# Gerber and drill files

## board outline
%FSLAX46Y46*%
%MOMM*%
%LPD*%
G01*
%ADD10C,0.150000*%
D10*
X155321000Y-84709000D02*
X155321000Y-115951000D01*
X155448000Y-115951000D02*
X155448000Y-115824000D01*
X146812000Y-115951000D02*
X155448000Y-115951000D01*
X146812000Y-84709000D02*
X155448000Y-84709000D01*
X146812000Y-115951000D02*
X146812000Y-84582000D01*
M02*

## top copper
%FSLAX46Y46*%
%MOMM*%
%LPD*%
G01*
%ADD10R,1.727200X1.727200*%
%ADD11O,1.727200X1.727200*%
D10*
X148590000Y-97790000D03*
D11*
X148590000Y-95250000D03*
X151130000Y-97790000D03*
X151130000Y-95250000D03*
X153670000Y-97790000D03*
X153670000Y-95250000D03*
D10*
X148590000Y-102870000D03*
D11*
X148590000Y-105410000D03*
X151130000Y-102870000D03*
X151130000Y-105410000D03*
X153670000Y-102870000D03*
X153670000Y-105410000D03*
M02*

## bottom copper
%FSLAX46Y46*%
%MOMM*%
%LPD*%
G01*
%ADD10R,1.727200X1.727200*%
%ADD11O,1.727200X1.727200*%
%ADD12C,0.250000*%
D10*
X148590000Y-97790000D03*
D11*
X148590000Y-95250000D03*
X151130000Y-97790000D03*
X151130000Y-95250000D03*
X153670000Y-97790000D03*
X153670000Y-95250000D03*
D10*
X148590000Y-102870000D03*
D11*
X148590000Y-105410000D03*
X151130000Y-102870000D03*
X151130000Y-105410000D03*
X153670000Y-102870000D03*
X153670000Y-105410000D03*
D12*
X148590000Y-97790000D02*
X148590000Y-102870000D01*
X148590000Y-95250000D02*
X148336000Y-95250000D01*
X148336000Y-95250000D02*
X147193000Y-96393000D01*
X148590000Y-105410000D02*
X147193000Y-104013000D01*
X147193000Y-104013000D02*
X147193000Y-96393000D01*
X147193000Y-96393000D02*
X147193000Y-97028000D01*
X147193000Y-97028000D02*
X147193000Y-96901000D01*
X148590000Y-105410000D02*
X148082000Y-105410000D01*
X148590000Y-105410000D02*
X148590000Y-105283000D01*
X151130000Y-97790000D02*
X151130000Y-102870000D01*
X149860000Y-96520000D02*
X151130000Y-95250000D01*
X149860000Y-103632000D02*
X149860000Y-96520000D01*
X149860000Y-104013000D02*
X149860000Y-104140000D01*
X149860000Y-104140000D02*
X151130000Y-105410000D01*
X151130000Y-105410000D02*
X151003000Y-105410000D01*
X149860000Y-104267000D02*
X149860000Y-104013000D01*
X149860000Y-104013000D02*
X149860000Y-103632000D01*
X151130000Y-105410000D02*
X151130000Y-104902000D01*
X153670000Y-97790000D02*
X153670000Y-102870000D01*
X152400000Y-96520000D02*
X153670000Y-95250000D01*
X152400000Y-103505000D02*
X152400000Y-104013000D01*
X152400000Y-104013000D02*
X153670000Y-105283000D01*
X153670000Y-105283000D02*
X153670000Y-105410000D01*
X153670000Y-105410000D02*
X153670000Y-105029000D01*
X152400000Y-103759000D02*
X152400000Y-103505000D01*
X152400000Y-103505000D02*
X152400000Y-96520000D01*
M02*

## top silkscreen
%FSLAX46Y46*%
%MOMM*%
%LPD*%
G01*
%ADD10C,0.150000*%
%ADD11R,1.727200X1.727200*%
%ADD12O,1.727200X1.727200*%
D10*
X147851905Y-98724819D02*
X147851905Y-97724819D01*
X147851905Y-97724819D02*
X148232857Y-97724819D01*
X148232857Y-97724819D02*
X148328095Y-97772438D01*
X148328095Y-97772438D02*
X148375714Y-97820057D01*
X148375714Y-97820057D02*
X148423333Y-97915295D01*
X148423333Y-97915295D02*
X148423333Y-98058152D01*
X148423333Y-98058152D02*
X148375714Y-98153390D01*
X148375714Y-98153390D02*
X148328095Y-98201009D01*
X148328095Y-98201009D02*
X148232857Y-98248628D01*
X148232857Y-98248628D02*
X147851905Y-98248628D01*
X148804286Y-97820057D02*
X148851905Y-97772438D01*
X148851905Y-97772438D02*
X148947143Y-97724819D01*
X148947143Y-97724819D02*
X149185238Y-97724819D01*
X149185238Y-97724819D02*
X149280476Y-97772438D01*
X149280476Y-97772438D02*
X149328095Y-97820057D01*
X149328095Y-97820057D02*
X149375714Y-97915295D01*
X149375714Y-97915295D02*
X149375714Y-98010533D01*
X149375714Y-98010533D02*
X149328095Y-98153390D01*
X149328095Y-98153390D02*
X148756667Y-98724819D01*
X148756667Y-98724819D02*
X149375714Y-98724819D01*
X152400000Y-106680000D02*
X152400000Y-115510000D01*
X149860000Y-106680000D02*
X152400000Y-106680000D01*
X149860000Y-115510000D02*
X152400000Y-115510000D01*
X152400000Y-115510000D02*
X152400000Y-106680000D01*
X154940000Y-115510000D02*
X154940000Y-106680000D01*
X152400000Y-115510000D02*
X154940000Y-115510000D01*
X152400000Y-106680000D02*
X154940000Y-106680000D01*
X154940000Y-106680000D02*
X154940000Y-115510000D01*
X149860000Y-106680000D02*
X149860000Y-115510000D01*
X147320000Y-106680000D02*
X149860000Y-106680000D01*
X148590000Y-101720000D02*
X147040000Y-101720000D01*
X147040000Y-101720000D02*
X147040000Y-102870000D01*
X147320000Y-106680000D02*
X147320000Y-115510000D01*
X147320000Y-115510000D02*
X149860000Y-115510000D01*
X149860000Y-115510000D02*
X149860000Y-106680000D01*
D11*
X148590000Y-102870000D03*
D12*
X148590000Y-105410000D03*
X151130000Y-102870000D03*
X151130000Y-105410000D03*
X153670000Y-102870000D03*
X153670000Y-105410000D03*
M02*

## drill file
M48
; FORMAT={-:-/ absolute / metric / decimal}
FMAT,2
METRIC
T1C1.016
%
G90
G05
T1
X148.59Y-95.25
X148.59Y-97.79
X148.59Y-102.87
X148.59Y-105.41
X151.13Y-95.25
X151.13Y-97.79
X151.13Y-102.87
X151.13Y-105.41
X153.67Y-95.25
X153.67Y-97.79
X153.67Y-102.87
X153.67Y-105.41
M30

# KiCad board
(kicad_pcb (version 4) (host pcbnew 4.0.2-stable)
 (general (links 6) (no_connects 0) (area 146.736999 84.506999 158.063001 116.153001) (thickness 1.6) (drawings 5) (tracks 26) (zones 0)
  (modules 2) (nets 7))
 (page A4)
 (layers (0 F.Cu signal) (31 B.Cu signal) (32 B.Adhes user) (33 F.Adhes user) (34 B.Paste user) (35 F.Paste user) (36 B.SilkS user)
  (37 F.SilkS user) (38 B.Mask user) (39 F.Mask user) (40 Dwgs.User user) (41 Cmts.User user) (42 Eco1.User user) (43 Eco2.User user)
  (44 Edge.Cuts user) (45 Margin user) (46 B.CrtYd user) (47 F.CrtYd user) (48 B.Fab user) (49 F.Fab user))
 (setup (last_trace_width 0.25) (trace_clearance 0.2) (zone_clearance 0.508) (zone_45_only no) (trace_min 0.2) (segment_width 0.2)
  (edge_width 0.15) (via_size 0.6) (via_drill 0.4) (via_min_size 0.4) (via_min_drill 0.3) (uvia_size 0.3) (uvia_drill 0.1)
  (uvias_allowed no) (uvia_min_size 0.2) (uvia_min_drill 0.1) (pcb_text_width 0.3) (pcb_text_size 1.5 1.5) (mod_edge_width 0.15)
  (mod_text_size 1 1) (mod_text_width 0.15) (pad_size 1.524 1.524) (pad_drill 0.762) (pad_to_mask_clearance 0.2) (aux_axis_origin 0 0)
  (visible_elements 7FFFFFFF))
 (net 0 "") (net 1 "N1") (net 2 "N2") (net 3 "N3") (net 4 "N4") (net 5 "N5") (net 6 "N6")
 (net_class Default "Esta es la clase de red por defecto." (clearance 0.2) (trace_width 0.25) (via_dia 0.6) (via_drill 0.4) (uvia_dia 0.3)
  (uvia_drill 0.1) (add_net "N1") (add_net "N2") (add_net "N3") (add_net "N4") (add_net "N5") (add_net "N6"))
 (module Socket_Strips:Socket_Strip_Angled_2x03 (layer B.Cu) (at 148.59 97.79)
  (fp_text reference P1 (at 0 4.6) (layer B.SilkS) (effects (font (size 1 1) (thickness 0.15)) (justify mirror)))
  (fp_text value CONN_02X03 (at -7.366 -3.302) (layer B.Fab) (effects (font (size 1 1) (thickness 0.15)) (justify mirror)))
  (pad 1 thru_hole rect (at 0 0) (size 1.7272 1.7272) (drill 1.016) (layers *.Cu *.Mask B.SilkS) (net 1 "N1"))
  (pad 2 thru_hole oval (at 0 -2.54) (size 1.7272 1.7272) (drill 1.016) (layers *.Cu *.Mask B.SilkS) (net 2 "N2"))
  (pad 3 thru_hole oval (at 2.54 0) (size 1.7272 1.7272) (drill 1.016) (layers *.Cu *.Mask B.SilkS) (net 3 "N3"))
  (pad 4 thru_hole oval (at 2.54 -2.54) (size 1.7272 1.7272) (drill 1.016) (layers *.Cu *.Mask B.SilkS) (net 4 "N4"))
  (pad 5 thru_hole oval (at 5.08 0) (size 1.7272 1.7272) (drill 1.016) (layers *.Cu *.Mask B.SilkS) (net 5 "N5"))
  (pad 6 thru_hole oval (at 5.08 -2.54) (size 1.7272 1.7272) (drill 1.016) (layers *.Cu *.Mask B.SilkS) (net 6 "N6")))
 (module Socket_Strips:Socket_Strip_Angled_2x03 (layer F.Cu) (at 148.59 102.87)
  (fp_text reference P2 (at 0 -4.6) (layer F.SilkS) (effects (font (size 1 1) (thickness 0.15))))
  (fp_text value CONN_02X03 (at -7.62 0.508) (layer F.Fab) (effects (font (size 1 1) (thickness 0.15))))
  (fp_line (start 3.81 3.81) (end 3.81 12.64) (layer F.SilkS) (width 0.15))
  (fp_line (start 1.27 3.81) (end 3.81 3.81) (layer F.SilkS) (width 0.15))
  (fp_line (start 1.27 12.64) (end 3.81 12.64) (layer F.SilkS) (width 0.15))
  (fp_line (start 3.81 12.64) (end 3.81 3.81) (layer F.SilkS) (width 0.15))
  (fp_line (start 6.35 12.64) (end 6.35 3.81) (layer F.SilkS) (width 0.15))
  (fp_line (start 3.81 12.64) (end 6.35 12.64) (layer F.SilkS) (width 0.15))
  (fp_line (start 3.81 3.81) (end 6.35 3.81) (layer F.SilkS) (width 0.15))
  (fp_line (start 6.35 3.81) (end 6.35 12.64) (layer F.SilkS) (width 0.15))
  (fp_line (start 1.27 3.81) (end 1.27 12.64) (layer F.SilkS) (width 0.15))
  (fp_line (start -1.27 3.81) (end 1.27 3.81) (layer F.SilkS) (width 0.15))
  (fp_line (start 0 -1.15) (end -1.55 -1.15) (layer F.SilkS) (width 0.15))
  (fp_line (start -1.55 -1.15) (end -1.55 0) (layer F.SilkS) (width 0.15))
  (fp_line (start -1.27 3.81) (end -1.27 12.64) (layer F.SilkS) (width 0.15))
  (fp_line (start -1.27 12.64) (end 1.27 12.64) (layer F.SilkS) (width 0.15))
  (fp_line (start 1.27 12.64) (end 1.27 3.81) (layer F.SilkS) (width 0.15))
  (pad 1 thru_hole rect (at 0 0) (size 1.7272 1.7272) (drill 1.016) (layers *.Cu *.Mask F.SilkS) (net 1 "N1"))
  (pad 2 thru_hole oval (at 0 2.54) (size 1.7272 1.7272) (drill 1.016) (layers *.Cu *.Mask F.SilkS) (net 2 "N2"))
  (pad 3 thru_hole oval (at 2.54 0) (size 1.7272 1.7272) (drill 1.016) (layers *.Cu *.Mask F.SilkS) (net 3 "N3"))
  (pad 4 thru_hole oval (at 2.54 2.54) (size 1.7272 1.7272) (drill 1.016) (layers *.Cu *.Mask F.SilkS) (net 4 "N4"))
  (pad 5 thru_hole oval (at 5.08 0) (size 1.7272 1.7272) (drill 1.016) (layers *.Cu *.Mask F.SilkS) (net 5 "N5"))
  (pad 6 thru_hole oval (at 5.08 2.54) (size 1.7272 1.7272) (drill 1.016) (layers *.Cu *.Mask F.SilkS) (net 6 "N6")))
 (gr_line (start 155.321 84.709) (end 155.321 115.951) (angle 90) (layer Edge.Cuts) (width 0.15))
 (gr_line (start 155.448 115.951) (end 155.448 115.824) (angle 90) (layer Edge.Cuts) (width 0.15))
 (gr_line (start 146.812 115.951) (end 155.448 115.951) (angle 90) (layer Edge.Cuts) (width 0.15))
 (gr_line (start 146.812 84.709) (end 155.448 84.709) (angle 90) (layer Edge.Cuts) (width 0.15))
 (gr_line (start 146.812 115.951) (end 146.812 84.582) (angle 90) (layer Edge.Cuts) (width 0.15))
 (segment (start 148.59 97.79) (end 148.59 102.87) (width 0.25) (layer B.Cu) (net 1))
 (segment (start 148.59 95.25) (end 148.336 95.25) (width 0.25) (layer B.Cu) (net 2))
 (segment (start 148.336 95.25) (end 147.193 96.393) (width 0.25) (layer B.Cu) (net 2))
 (segment (start 148.59 105.41) (end 147.193 104.013) (width 0.25) (layer B.Cu) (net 2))
 (segment (start 147.193 104.013) (end 147.193 96.393) (width 0.25) (layer B.Cu) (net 2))
 (segment (start 147.193 96.393) (end 147.193 97.028) (width 0.25) (layer B.Cu) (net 2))
 (segment (start 147.193 97.028) (end 147.193 96.901) (width 0.25) (layer B.Cu) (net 2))
 (segment (start 148.59 105.41) (end 148.082 105.41) (width 0.25) (layer B.Cu) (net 2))
 (segment (start 148.59 105.41) (end 148.59 105.283) (width 0.25) (layer B.Cu) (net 2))
 (segment (start 151.13 97.79) (end 151.13 102.87) (width 0.25) (layer B.Cu) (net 3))
 (segment (start 149.86 96.52) (end 151.13 95.25) (width 0.25) (layer B.Cu) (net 4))
 (segment (start 149.86 103.632) (end 149.86 96.52) (width 0.25) (layer B.Cu) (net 4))
 (segment (start 149.86 104.013) (end 149.86 104.14) (width 0.25) (layer B.Cu) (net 4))
 (segment (start 149.86 104.14) (end 151.13 105.41) (width 0.25) (layer B.Cu) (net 4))
 (segment (start 151.13 105.41) (end 151.003 105.41) (width 0.25) (layer B.Cu) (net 4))
 (segment (start 149.86 104.267) (end 149.86 104.013) (width 0.25) (layer B.Cu) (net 4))
 (segment (start 149.86 104.013) (end 149.86 103.632) (width 0.25) (layer B.Cu) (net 4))
 (segment (start 151.13 105.41) (end 151.13 104.902) (width 0.25) (layer B.Cu) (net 4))
 (segment (start 153.67 97.79) (end 153.67 102.87) (width 0.25) (layer B.Cu) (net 5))
 (segment (start 152.4 96.52) (end 153.67 95.25) (width 0.25) (layer B.Cu) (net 6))
 (segment (start 152.4 103.505) (end 152.4 104.013) (width 0.25) (layer B.Cu) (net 6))
 (segment (start 152.4 104.013) (end 153.67 105.283) (width 0.25) (layer B.Cu) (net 6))
 (segment (start 153.67 105.283) (end 153.67 105.41) (width 0.25) (layer B.Cu) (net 6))
 (segment (start 153.67 105.41) (end 153.67 105.029) (width 0.25) (layer B.Cu) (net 6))
 (segment (start 152.4 103.759) (end 152.4 103.505) (width 0.25) (layer B.Cu) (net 6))
 (segment (start 152.4 103.505) (end 152.4 96.52) (width 0.25) (layer B.Cu) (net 6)))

